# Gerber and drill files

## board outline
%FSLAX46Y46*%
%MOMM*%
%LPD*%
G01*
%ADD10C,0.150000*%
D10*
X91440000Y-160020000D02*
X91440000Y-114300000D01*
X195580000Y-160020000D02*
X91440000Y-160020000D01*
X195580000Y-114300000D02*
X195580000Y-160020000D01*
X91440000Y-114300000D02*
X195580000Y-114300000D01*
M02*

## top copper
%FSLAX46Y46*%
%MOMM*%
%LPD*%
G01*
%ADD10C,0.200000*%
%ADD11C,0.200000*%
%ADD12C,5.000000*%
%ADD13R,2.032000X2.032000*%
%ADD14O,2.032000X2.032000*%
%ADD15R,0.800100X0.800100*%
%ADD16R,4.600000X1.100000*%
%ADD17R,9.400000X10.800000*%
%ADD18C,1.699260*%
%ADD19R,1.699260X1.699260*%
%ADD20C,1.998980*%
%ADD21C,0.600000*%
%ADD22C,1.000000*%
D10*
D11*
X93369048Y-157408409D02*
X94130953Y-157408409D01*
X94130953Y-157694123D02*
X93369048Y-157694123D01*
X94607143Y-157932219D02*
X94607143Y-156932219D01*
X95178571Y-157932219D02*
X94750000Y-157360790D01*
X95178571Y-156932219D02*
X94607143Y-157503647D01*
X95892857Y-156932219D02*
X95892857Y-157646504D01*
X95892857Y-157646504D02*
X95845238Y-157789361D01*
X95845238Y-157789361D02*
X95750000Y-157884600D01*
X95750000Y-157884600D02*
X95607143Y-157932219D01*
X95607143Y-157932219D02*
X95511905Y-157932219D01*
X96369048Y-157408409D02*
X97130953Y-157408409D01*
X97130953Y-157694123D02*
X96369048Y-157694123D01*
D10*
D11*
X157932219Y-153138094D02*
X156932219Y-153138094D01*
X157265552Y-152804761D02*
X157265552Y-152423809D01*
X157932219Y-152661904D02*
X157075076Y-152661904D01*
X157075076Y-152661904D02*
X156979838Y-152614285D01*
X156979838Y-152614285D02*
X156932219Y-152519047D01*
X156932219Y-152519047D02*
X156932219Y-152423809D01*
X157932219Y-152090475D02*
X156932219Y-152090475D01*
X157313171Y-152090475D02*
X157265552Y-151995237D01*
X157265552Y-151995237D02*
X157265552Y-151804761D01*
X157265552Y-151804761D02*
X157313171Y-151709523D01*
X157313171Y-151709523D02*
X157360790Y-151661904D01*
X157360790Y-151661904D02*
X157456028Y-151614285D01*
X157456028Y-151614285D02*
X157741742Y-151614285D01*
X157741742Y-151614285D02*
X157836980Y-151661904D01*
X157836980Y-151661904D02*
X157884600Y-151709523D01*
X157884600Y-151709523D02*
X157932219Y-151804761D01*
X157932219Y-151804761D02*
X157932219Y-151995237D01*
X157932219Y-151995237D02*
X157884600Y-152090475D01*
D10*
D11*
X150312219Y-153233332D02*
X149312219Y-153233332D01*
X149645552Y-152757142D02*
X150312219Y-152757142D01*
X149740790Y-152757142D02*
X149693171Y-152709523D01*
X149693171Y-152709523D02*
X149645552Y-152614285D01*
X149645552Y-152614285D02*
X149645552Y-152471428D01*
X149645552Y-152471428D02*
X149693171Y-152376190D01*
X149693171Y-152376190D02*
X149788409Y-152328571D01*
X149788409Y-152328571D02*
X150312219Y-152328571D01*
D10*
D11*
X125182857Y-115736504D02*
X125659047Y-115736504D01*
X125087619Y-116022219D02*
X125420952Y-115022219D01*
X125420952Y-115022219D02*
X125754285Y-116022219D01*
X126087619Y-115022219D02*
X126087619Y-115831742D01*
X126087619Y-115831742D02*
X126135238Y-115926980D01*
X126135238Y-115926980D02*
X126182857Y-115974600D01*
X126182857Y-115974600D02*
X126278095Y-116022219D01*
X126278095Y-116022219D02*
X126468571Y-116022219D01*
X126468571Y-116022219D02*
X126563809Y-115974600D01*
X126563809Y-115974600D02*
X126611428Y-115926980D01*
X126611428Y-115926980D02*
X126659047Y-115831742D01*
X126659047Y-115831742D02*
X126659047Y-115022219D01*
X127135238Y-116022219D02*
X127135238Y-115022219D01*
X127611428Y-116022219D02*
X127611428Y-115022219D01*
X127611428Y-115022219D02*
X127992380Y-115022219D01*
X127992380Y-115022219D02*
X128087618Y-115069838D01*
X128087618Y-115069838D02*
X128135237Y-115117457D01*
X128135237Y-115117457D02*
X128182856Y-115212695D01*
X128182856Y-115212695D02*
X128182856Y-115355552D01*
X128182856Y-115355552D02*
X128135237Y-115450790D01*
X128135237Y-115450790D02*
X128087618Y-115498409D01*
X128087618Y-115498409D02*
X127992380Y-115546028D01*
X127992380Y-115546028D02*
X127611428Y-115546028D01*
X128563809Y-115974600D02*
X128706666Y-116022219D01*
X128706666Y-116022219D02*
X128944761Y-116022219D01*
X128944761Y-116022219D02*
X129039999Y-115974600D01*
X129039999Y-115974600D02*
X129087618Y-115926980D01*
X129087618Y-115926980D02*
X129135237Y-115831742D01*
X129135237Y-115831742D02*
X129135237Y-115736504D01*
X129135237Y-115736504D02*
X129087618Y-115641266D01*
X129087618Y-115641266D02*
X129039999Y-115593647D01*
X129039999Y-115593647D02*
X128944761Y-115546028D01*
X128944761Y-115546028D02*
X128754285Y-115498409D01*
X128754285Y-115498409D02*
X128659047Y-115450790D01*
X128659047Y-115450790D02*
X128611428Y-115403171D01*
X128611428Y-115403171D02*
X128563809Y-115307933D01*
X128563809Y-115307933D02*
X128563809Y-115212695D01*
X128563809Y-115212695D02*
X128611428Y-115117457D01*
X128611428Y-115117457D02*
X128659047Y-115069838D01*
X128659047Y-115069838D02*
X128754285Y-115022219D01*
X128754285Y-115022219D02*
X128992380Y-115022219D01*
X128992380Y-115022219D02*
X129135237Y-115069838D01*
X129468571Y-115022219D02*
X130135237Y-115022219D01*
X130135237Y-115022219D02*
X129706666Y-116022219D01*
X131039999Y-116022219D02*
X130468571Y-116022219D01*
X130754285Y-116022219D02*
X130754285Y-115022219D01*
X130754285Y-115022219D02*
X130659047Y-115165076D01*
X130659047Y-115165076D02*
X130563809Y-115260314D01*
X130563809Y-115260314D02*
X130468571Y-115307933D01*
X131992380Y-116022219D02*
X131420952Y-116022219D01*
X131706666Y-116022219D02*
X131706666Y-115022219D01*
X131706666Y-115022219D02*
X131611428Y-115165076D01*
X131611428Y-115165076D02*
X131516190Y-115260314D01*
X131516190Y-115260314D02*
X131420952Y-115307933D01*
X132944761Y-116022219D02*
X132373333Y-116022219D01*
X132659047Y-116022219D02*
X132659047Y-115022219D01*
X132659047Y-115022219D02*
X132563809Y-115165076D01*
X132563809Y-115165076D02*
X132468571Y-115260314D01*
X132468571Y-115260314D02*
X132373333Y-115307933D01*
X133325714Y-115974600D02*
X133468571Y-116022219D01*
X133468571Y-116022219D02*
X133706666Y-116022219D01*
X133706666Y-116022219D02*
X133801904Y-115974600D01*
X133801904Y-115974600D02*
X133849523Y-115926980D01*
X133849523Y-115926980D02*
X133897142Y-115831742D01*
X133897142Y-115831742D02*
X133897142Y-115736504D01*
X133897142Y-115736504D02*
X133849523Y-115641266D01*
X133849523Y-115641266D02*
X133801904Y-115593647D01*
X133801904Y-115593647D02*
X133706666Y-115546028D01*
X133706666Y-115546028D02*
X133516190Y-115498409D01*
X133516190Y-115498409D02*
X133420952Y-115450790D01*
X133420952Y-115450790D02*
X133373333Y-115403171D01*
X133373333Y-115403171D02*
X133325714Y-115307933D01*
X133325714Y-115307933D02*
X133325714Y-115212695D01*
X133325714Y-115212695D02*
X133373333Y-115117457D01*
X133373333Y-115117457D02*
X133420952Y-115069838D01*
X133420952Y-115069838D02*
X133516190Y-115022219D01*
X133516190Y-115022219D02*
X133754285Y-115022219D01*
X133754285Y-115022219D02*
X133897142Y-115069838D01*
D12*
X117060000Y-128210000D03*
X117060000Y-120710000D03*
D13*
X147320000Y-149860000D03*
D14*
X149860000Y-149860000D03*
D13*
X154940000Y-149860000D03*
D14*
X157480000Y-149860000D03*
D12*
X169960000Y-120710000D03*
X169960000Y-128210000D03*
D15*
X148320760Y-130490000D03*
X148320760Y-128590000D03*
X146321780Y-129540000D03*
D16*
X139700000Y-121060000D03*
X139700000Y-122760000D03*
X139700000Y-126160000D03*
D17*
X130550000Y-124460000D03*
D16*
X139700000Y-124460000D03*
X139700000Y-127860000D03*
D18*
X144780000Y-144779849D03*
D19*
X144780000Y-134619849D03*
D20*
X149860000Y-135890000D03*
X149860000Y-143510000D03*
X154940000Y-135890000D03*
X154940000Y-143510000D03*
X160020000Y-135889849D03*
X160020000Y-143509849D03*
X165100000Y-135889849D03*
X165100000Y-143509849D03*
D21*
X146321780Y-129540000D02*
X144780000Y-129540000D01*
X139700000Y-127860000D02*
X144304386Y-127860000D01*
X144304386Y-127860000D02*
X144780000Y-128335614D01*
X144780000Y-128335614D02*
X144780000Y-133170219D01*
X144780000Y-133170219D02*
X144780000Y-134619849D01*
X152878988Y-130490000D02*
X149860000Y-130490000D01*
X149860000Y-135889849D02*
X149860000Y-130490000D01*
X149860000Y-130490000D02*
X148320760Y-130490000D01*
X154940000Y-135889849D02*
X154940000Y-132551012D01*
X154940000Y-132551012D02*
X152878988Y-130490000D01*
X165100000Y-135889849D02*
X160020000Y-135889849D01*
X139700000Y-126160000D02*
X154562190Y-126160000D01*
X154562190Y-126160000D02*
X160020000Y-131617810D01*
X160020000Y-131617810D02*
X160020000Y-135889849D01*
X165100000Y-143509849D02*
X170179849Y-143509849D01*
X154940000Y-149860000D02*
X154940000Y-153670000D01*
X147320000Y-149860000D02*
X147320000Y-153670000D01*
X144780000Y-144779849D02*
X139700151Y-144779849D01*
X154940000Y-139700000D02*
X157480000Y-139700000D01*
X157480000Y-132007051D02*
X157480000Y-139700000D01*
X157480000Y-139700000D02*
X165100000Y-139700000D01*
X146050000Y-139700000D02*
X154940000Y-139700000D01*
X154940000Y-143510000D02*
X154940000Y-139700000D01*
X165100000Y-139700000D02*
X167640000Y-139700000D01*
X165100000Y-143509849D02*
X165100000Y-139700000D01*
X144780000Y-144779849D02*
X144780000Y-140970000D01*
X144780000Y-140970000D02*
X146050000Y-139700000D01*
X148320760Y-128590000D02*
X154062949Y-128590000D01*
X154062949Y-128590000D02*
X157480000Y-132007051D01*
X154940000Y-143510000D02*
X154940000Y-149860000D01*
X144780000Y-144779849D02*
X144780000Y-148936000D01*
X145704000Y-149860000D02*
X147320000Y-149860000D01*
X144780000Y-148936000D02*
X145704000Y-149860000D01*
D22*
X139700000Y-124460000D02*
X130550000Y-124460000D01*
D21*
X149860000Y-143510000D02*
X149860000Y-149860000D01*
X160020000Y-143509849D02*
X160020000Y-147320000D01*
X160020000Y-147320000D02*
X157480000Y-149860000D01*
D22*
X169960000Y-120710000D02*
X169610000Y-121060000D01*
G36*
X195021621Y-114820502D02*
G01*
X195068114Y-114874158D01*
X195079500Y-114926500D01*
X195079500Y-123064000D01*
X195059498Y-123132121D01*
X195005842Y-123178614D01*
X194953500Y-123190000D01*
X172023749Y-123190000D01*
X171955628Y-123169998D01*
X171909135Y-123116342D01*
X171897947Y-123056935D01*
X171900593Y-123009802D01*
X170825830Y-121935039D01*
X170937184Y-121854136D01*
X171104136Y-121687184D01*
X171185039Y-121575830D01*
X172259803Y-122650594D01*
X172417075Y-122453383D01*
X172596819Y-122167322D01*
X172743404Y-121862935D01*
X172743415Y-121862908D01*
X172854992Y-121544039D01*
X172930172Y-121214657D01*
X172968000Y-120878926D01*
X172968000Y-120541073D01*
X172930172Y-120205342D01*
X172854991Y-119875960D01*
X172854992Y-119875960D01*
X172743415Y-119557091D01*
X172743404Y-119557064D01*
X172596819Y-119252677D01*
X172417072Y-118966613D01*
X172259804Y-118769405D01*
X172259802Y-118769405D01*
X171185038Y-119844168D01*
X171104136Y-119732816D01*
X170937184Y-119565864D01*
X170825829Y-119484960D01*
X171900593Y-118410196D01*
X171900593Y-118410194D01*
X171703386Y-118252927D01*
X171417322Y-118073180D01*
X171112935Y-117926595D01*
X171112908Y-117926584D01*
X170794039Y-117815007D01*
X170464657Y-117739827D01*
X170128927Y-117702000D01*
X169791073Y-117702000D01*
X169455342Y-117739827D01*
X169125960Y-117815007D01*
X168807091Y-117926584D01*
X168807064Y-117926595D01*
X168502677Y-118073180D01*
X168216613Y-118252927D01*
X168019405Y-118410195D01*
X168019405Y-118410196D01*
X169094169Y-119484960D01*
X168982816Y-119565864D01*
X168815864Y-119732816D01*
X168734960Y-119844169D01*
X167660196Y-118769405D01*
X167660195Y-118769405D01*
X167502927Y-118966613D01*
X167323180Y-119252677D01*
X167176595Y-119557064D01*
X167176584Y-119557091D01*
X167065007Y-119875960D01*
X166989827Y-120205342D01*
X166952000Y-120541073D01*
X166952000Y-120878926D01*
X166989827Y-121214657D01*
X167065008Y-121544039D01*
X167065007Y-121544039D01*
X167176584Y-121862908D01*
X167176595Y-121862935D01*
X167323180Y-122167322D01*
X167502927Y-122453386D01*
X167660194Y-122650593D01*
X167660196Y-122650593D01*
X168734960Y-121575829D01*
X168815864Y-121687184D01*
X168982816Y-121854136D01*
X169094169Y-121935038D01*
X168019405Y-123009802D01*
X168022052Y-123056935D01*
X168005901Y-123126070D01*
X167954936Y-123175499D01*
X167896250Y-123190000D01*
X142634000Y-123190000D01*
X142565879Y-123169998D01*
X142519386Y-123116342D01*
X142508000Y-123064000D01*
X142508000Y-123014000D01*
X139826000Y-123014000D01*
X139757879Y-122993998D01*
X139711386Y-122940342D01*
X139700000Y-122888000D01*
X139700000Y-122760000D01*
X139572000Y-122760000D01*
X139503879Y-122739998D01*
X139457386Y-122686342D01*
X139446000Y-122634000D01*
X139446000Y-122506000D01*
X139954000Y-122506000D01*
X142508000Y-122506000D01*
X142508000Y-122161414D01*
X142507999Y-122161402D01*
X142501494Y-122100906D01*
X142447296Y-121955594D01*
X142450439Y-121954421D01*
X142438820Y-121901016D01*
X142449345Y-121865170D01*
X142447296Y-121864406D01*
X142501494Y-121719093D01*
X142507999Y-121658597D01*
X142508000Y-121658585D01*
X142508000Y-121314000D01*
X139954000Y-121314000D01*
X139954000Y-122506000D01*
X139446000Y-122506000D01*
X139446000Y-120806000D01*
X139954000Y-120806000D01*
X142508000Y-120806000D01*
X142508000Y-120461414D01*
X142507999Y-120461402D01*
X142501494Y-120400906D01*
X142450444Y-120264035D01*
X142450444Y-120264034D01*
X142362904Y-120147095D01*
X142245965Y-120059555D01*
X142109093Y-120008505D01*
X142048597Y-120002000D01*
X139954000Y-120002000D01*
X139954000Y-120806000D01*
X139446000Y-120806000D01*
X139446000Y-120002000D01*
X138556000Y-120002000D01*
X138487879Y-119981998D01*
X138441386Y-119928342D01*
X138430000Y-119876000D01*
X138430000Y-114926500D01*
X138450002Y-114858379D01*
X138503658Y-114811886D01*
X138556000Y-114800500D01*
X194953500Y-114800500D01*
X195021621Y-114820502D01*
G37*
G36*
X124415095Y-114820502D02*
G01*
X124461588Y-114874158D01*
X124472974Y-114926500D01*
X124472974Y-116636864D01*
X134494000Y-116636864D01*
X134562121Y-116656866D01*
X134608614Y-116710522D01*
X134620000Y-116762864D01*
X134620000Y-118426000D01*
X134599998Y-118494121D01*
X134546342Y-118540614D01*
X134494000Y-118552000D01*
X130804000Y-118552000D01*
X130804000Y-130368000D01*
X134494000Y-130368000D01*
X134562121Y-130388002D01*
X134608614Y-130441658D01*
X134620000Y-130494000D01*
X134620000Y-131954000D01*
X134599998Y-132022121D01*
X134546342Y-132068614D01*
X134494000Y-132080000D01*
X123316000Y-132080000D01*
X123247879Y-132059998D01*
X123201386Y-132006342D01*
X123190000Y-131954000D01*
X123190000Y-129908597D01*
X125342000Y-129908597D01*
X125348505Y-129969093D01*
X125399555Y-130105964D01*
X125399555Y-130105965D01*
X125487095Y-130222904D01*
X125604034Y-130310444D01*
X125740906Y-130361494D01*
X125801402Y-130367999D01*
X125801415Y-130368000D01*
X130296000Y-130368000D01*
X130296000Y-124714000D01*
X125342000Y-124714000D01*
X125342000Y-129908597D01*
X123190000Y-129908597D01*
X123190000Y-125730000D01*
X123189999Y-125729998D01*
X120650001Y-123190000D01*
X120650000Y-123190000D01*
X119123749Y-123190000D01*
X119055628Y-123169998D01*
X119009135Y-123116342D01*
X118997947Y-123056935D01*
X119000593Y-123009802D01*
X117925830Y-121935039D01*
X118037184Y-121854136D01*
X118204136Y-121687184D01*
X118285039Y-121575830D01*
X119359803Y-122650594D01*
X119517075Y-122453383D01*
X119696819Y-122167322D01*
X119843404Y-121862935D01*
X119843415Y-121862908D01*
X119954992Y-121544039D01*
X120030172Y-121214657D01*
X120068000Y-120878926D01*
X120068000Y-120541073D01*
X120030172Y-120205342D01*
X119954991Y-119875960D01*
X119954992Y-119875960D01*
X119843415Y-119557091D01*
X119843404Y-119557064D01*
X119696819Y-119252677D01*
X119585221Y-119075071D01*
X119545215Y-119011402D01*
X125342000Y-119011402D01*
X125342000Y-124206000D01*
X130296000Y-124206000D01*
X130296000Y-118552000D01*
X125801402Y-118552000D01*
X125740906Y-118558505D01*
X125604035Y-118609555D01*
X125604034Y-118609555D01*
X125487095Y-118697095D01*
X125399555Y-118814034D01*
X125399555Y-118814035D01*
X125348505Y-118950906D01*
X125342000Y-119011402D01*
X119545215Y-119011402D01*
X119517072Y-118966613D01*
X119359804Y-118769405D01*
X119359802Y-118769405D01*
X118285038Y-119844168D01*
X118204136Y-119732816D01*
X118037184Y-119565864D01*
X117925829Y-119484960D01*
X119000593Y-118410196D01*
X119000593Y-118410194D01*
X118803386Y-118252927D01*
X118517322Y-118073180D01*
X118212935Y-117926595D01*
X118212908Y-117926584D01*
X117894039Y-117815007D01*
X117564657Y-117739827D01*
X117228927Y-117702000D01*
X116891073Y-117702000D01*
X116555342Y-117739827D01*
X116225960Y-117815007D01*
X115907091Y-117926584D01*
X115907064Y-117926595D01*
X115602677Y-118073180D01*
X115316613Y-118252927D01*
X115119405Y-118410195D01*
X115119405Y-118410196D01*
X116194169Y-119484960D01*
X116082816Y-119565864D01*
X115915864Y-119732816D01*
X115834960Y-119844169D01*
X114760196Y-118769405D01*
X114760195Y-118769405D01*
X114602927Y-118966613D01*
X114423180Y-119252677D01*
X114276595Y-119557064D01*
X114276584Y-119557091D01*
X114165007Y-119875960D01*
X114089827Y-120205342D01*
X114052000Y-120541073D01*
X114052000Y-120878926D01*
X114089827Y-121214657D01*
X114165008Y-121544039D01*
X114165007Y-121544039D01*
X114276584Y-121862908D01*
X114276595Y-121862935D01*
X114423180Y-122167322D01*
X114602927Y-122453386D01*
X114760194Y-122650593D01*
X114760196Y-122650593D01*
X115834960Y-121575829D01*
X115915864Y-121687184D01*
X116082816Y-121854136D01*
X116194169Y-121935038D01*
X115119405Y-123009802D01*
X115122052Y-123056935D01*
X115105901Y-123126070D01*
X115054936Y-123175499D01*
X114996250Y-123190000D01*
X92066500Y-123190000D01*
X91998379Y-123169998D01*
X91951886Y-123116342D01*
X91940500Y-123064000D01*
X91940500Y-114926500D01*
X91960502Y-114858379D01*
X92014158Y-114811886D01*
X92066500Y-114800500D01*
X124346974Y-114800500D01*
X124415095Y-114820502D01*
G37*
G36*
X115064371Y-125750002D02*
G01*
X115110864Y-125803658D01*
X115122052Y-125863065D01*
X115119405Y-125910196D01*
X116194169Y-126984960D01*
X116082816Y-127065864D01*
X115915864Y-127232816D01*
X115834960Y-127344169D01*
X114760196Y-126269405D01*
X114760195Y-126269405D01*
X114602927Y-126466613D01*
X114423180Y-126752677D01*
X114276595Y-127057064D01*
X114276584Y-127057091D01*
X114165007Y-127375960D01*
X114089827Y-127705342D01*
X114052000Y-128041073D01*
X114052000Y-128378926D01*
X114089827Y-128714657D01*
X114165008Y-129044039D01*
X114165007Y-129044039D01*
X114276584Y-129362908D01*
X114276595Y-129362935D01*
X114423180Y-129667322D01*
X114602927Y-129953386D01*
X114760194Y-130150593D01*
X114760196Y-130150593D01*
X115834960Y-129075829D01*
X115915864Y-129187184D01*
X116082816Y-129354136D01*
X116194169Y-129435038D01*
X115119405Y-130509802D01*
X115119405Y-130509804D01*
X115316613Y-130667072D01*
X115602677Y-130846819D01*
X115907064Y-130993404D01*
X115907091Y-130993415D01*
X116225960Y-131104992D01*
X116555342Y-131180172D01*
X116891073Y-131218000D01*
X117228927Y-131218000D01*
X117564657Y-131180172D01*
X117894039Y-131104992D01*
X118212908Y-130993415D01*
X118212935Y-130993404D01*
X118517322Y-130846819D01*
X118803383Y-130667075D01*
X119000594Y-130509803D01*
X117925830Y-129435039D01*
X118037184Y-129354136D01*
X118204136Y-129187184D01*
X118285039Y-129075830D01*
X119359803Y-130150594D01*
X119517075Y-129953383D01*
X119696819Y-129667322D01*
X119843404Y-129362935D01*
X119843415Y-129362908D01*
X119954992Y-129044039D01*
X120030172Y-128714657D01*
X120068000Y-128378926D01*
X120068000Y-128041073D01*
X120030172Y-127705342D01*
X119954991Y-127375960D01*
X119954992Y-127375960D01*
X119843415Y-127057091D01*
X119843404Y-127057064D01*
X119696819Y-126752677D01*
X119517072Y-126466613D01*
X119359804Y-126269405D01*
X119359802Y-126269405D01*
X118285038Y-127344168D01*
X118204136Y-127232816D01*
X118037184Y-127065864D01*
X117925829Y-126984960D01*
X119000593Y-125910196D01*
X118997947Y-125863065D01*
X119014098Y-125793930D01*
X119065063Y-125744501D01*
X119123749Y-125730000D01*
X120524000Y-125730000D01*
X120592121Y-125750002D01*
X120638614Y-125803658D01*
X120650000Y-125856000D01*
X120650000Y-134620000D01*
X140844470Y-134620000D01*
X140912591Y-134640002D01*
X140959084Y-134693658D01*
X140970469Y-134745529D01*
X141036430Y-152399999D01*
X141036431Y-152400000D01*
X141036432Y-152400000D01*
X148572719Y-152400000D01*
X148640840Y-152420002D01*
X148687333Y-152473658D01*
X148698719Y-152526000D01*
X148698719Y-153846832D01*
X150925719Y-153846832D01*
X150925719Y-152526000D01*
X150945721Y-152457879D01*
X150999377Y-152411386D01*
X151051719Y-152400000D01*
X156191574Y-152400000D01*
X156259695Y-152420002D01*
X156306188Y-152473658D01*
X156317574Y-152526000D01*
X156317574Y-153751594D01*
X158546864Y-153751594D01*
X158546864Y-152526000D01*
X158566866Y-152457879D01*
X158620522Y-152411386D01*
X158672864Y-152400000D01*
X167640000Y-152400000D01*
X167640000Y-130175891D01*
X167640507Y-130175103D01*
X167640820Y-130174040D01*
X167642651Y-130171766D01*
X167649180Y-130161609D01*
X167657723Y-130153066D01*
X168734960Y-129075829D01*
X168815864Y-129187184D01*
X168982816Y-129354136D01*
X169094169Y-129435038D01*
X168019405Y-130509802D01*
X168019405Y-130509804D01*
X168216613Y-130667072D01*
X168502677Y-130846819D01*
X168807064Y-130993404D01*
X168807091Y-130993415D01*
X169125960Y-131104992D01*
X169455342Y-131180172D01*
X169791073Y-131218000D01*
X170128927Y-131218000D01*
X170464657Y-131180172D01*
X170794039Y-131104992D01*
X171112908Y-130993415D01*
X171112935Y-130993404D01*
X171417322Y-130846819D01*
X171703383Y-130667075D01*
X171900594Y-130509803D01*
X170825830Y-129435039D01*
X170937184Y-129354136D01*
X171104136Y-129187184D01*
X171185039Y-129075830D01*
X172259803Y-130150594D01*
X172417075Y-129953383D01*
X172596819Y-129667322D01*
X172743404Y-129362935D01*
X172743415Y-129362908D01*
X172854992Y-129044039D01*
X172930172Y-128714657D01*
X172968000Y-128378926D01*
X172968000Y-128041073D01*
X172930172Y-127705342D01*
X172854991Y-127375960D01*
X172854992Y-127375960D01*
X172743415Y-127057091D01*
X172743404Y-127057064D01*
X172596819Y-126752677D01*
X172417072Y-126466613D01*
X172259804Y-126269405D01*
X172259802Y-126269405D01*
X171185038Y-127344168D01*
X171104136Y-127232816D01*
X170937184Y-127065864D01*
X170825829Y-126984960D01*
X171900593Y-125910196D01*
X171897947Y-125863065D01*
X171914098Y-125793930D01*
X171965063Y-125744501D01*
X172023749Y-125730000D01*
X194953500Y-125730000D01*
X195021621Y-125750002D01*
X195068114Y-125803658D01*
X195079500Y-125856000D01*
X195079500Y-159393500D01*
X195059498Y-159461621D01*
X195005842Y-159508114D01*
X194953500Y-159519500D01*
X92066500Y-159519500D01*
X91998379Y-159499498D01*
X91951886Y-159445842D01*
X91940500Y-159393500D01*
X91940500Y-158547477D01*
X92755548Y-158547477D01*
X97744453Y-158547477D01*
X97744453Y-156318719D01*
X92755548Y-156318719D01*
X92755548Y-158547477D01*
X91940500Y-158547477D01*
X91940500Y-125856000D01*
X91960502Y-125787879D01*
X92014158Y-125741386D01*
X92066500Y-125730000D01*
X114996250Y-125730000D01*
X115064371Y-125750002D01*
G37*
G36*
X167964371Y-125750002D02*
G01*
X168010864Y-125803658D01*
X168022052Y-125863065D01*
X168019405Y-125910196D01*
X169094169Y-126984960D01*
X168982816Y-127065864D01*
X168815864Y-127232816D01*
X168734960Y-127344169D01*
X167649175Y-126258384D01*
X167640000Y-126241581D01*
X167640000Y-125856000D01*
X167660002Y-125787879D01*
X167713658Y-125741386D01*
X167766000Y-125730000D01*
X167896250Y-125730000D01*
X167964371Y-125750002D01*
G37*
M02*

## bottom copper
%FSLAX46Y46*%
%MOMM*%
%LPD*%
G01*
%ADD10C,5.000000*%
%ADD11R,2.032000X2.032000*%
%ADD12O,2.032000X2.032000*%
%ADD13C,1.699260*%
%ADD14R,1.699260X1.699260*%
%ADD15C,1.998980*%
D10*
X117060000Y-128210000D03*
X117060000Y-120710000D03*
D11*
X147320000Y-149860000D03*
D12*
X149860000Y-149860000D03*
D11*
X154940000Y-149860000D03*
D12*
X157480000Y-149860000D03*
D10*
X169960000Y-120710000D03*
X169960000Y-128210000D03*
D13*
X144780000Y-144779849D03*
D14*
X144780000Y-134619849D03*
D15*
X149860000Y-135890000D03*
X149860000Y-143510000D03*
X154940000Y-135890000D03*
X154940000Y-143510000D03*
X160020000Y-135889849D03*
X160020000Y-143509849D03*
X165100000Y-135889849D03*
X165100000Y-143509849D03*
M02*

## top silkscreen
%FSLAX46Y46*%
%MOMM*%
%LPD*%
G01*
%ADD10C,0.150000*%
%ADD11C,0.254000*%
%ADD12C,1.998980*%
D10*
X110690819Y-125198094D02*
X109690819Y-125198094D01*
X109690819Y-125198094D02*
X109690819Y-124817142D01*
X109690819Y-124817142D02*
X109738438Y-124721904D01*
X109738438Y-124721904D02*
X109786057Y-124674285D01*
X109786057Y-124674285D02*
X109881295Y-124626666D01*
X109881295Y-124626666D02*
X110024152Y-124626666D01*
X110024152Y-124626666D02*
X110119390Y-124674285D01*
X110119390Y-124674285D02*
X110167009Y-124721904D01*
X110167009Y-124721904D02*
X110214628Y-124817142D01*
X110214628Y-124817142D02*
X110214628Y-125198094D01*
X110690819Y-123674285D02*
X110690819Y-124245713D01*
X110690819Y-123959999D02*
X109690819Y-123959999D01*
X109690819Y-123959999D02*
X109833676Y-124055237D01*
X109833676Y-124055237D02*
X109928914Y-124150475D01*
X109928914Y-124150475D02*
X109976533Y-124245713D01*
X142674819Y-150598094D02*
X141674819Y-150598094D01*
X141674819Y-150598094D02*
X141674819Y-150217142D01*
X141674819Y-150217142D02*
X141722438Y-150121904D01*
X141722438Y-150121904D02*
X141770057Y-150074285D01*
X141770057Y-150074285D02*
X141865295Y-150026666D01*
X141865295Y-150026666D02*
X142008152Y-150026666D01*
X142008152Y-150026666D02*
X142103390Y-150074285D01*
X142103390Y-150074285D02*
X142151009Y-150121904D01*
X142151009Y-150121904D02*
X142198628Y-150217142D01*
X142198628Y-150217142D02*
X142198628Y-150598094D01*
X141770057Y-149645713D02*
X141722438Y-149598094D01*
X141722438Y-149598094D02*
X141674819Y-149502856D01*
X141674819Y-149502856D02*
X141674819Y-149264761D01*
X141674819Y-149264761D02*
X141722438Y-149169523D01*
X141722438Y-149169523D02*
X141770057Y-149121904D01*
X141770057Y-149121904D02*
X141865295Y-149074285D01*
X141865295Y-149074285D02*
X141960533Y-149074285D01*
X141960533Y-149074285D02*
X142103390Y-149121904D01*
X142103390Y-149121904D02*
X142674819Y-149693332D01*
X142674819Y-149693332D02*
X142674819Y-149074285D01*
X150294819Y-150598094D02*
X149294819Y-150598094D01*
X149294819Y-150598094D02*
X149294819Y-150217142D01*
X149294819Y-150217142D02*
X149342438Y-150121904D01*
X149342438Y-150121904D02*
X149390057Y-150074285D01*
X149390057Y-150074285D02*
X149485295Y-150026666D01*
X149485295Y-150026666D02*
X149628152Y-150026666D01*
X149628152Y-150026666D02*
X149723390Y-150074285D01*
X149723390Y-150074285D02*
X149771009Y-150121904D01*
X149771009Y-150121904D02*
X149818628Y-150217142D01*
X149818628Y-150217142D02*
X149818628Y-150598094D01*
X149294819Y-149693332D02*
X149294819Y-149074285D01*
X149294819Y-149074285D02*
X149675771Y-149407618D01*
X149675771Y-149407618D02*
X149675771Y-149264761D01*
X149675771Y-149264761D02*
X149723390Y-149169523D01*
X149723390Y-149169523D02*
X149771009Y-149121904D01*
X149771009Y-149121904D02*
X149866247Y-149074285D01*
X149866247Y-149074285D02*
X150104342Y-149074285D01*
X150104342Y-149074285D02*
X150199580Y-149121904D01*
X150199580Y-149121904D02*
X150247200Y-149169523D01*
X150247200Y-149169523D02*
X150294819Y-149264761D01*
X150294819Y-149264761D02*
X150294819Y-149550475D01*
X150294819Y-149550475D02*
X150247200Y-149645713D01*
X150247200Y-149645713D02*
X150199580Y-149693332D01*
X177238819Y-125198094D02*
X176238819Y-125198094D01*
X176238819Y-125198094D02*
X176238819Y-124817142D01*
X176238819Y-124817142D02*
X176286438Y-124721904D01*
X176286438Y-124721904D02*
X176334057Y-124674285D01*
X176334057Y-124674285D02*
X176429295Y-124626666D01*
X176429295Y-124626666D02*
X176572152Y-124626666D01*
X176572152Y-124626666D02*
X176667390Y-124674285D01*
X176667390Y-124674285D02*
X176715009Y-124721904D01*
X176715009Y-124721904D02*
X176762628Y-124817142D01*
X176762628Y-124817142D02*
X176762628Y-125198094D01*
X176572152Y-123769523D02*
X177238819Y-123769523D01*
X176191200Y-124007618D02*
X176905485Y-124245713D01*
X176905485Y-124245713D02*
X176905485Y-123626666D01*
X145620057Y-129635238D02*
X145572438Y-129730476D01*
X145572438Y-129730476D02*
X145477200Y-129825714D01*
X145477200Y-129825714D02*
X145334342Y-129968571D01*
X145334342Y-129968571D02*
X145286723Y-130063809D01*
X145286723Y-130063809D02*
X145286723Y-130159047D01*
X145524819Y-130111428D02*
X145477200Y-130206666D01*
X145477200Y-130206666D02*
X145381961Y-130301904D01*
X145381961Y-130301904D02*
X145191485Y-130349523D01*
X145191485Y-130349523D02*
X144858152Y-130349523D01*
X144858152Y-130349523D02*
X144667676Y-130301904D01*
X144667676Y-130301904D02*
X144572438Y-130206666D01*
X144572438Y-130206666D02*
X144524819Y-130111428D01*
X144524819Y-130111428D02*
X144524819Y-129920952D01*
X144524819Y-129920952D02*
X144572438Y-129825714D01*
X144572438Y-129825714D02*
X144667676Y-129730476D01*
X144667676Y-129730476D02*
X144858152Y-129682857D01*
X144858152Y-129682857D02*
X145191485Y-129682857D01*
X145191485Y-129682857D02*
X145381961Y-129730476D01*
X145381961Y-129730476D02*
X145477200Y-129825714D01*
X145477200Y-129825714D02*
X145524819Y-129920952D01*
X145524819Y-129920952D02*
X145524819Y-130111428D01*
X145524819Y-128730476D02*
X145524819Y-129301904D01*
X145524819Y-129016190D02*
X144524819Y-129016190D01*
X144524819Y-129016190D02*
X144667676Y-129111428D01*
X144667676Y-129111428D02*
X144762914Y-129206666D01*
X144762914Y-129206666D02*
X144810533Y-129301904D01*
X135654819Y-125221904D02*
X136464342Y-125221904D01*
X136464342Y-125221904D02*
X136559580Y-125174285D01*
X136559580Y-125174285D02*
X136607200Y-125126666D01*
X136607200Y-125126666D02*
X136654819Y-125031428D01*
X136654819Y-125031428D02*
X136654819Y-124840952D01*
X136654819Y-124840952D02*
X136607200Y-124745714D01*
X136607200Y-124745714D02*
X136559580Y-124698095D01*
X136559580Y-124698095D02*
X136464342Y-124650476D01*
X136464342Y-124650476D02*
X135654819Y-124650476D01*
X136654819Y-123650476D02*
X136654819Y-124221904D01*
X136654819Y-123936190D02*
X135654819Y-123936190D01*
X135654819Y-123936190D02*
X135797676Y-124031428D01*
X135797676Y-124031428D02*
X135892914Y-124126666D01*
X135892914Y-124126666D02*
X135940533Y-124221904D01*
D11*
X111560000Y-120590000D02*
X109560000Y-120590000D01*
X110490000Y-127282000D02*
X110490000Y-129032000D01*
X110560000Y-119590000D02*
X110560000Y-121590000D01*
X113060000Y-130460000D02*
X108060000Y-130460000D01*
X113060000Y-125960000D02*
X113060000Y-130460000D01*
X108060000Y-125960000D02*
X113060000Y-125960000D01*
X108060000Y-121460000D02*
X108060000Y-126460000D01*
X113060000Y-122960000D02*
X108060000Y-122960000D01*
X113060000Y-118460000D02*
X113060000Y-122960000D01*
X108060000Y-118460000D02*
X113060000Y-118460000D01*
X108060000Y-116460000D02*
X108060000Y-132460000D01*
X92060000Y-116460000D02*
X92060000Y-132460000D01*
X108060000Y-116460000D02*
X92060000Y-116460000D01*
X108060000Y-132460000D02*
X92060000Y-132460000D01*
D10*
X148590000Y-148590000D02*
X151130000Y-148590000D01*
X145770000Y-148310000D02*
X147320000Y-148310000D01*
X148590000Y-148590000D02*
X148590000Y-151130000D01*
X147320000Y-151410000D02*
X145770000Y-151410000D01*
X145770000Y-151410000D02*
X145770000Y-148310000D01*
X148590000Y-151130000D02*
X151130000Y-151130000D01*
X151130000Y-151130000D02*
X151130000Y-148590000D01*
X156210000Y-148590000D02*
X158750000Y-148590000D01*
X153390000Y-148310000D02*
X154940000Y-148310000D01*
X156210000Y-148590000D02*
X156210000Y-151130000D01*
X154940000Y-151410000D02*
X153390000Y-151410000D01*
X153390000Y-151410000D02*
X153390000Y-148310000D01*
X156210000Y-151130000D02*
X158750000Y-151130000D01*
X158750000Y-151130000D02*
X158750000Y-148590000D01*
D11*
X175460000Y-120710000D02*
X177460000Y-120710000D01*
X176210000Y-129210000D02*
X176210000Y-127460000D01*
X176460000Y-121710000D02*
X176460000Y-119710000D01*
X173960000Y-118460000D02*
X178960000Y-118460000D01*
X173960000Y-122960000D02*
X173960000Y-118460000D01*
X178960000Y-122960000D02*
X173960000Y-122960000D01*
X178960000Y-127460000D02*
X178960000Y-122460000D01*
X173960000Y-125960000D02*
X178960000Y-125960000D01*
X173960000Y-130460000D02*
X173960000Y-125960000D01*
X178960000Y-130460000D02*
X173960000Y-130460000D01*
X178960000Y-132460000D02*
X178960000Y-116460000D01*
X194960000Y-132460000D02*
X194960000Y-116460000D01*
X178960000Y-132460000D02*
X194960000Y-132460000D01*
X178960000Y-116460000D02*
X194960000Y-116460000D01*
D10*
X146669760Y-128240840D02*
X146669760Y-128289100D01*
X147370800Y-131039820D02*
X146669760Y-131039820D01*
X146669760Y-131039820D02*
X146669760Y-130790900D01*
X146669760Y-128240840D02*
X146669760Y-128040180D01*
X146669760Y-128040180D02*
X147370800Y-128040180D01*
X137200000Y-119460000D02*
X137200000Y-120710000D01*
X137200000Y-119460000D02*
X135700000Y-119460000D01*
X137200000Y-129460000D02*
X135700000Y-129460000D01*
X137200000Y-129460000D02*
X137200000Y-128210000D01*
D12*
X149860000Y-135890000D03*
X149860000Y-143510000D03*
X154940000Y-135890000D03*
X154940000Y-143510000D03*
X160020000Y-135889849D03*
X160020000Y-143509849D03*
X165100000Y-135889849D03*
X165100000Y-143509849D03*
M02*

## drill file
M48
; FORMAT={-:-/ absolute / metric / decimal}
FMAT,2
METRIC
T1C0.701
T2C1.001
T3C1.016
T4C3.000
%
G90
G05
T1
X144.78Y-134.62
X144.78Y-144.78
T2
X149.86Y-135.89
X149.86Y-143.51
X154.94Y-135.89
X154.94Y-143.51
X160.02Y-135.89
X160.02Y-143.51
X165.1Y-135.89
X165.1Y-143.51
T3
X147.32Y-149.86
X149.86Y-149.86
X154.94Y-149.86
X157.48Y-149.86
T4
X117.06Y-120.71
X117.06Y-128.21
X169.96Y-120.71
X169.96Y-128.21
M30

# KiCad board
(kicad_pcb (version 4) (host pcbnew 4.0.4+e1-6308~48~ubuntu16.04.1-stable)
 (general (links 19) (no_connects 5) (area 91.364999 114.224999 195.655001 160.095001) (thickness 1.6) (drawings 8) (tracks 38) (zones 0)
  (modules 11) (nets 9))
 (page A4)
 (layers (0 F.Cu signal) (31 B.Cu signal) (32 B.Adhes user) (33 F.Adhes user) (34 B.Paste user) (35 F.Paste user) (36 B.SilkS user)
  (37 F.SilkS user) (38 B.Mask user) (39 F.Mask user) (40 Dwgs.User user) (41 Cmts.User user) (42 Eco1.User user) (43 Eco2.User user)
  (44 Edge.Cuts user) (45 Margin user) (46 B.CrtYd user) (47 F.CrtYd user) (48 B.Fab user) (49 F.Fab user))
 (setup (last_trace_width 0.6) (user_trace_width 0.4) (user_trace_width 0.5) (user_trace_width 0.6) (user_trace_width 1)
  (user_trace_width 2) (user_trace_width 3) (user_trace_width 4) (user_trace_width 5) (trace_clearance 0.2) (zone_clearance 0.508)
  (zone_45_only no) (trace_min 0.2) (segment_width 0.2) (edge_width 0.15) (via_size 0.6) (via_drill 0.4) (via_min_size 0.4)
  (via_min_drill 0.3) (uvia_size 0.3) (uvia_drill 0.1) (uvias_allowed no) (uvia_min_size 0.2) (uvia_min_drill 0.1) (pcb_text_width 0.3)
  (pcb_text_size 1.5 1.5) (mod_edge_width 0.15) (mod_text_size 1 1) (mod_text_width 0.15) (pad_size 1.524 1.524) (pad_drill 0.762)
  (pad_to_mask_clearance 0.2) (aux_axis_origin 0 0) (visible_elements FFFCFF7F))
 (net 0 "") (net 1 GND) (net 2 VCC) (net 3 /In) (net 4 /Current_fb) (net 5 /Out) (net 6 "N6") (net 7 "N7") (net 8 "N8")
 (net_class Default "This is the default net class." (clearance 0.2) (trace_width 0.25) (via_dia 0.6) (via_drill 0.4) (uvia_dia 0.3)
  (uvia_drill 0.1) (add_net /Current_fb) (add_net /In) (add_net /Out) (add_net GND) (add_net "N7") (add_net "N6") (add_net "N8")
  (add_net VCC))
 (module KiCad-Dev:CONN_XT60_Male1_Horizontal (layer F.Cu) (at 99.06 124.46 270)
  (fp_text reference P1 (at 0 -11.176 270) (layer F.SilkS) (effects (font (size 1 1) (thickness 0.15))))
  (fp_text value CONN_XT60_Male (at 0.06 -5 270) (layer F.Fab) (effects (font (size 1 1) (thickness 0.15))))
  (fp_line (start -3.87 -12.5) (end -3.87 -10.5) (layer F.SilkS) (width 0.254))
  (fp_line (start 2.822 -11.43) (end 4.572 -11.43) (layer F.SilkS) (width 0.254))
  (fp_line (start -4.87 -11.5) (end -2.87 -11.5) (layer F.SilkS) (width 0.254))
  (fp_line (start 6 -14) (end 6 -9) (layer F.SilkS) (width 0.254))
  (fp_line (start 1.5 -14) (end 6 -14) (layer F.SilkS) (width 0.254))
  (fp_line (start 1.5 -9) (end 1.5 -14) (layer F.SilkS) (width 0.254))
  (fp_line (start -3 -9) (end 2 -9) (layer F.SilkS) (width 0.254))
  (fp_line (start -1.5 -14) (end -1.5 -9) (layer F.SilkS) (width 0.254))
  (fp_line (start -6 -14) (end -1.5 -14) (layer F.SilkS) (width 0.254))
  (fp_line (start -6 -9) (end -6 -14) (layer F.SilkS) (width 0.254))
  (fp_line (start -8 -9) (end 8 -9) (layer F.SilkS) (width 0.254))
  (fp_line (start -8 7) (end 8 7) (layer F.SilkS) (width 0.254))
  (fp_line (start -8 -9) (end -8 7) (layer F.SilkS) (width 0.254))
  (fp_line (start 8 -9) (end 8 7) (layer F.SilkS) (width 0.254))
  (pad 1 thru_hole circle (at 3.75 -18 270) (size 5 5) (drill 3) (layers *.Cu *.Mask) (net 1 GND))
  (pad 2 thru_hole circle (at -3.75 -18 270) (size 5 5) (drill 3) (layers *.Cu *.Mask) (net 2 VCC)))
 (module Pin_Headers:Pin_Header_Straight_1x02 (layer F.Cu) (at 147.32 149.86 90)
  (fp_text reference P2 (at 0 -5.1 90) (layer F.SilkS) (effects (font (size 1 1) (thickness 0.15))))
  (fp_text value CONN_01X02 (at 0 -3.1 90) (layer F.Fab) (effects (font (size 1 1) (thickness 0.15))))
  (fp_line (start 1.27 1.27) (end 1.27 3.81) (layer F.SilkS) (width 0.15))
  (fp_line (start 1.55 -1.55) (end 1.55 0) (layer F.SilkS) (width 0.15))
  (fp_line (start 1.27 1.27) (end -1.27 1.27) (layer F.SilkS) (width 0.15))
  (fp_line (start -1.55 0) (end -1.55 -1.55) (layer F.SilkS) (width 0.15))
  (fp_line (start -1.55 -1.55) (end 1.55 -1.55) (layer F.SilkS) (width 0.15))
  (fp_line (start -1.27 1.27) (end -1.27 3.81) (layer F.SilkS) (width 0.15))
  (fp_line (start -1.27 3.81) (end 1.27 3.81) (layer F.SilkS) (width 0.15))
  (pad 1 thru_hole rect (at 0 0 90) (size 2.032 2.032) (drill 1.016) (layers *.Cu *.Mask) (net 1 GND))
  (pad 2 thru_hole oval (at 0 2.54 90) (size 2.032 2.032) (drill 1.016) (layers *.Cu *.Mask) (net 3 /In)))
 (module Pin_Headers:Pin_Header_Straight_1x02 (layer F.Cu) (at 154.94 149.86 90)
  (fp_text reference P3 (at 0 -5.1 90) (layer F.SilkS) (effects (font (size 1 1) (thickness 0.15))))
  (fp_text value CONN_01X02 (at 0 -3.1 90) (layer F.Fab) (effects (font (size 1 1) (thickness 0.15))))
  (fp_line (start 1.27 1.27) (end 1.27 3.81) (layer F.SilkS) (width 0.15))
  (fp_line (start 1.55 -1.55) (end 1.55 0) (layer F.SilkS) (width 0.15))
  (fp_line (start 1.27 1.27) (end -1.27 1.27) (layer F.SilkS) (width 0.15))
  (fp_line (start -1.55 0) (end -1.55 -1.55) (layer F.SilkS) (width 0.15))
  (fp_line (start -1.55 -1.55) (end 1.55 -1.55) (layer F.SilkS) (width 0.15))
  (fp_line (start -1.27 1.27) (end -1.27 3.81) (layer F.SilkS) (width 0.15))
  (fp_line (start -1.27 3.81) (end 1.27 3.81) (layer F.SilkS) (width 0.15))
  (pad 1 thru_hole rect (at 0 0 90) (size 2.032 2.032) (drill 1.016) (layers *.Cu *.Mask) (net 1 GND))
  (pad 2 thru_hole oval (at 0 2.54 90) (size 2.032 2.032) (drill 1.016) (layers *.Cu *.Mask) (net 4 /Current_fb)))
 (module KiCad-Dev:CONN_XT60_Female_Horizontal (layer F.Cu) (at 187.96 124.46 90)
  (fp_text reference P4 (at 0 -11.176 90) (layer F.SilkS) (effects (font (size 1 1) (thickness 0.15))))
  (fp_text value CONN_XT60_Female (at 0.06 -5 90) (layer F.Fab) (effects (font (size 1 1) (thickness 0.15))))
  (fp_line (start 3.75 -12.5) (end 3.75 -10.5) (layer F.SilkS) (width 0.254))
  (fp_line (start -4.75 -11.75) (end -3 -11.75) (layer F.SilkS) (width 0.254))
  (fp_line (start 2.75 -11.5) (end 4.75 -11.5) (layer F.SilkS) (width 0.254))
  (fp_line (start 6 -14) (end 6 -9) (layer F.SilkS) (width 0.254))
  (fp_line (start 1.5 -14) (end 6 -14) (layer F.SilkS) (width 0.254))
  (fp_line (start 1.5 -9) (end 1.5 -14) (layer F.SilkS) (width 0.254))
  (fp_line (start -3 -9) (end 2 -9) (layer F.SilkS) (width 0.254))
  (fp_line (start -1.5 -14) (end -1.5 -9) (layer F.SilkS) (width 0.254))
  (fp_line (start -6 -14) (end -1.5 -14) (layer F.SilkS) (width 0.254))
  (fp_line (start -6 -9) (end -6 -14) (layer F.SilkS) (width 0.254))
  (fp_line (start -8 -9) (end 8 -9) (layer F.SilkS) (width 0.254))
  (fp_line (start -8 7) (end 8 7) (layer F.SilkS) (width 0.254))
  (fp_line (start -8 -9) (end -8 7) (layer F.SilkS) (width 0.254))
  (fp_line (start 8 -9) (end 8 7) (layer F.SilkS) (width 0.254))
  (pad 2 thru_hole circle (at 3.75 -18 90) (size 5 5) (drill 3) (layers *.Cu *.Mask) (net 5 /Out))
  (pad 1 thru_hole circle (at -3.75 -18 90) (size 5 5) (drill 3) (layers *.Cu *.Mask) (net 1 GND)))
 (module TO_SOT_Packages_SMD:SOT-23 (layer F.Cu) (at 147.32 129.54 90)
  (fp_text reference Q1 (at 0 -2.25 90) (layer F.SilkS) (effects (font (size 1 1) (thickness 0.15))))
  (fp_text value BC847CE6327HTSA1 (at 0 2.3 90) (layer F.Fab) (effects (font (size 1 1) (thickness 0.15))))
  (fp_line (start 1.29916 -0.65024) (end 1.2509 -0.65024) (layer F.SilkS) (width 0.15))
  (fp_line (start -1.49982 0.0508) (end -1.49982 -0.65024) (layer F.SilkS) (width 0.15))
  (fp_line (start -1.49982 -0.65024) (end -1.2509 -0.65024) (layer F.SilkS) (width 0.15))
  (fp_line (start 1.29916 -0.65024) (end 1.49982 -0.65024) (layer F.SilkS) (width 0.15))
  (fp_line (start 1.49982 -0.65024) (end 1.49982 0.0508) (layer F.SilkS) (width 0.15))
  (pad 1 smd rect (at -0.95 1.00076 90) (size 0.8001 0.8001) (layers F.Cu F.Paste F.Mask) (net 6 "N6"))
  (pad 2 smd rect (at 0.95 1.00076 90) (size 0.8001 0.8001) (layers F.Cu F.Paste F.Mask) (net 1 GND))
  (pad 3 smd rect (at 0 -0.99822 90) (size 0.8001 0.8001) (layers F.Cu F.Paste F.Mask) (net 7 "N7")))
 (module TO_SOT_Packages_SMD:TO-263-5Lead (layer F.Cu) (at 139.7 124.46 180)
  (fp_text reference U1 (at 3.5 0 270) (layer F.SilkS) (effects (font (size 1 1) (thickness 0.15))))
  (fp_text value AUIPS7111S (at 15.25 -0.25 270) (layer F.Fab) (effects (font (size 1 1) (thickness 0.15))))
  (fp_line (start 2.5 5) (end 2.5 3.75) (layer F.SilkS) (width 0.15))
  (fp_line (start 2.5 5) (end 4 5) (layer F.SilkS) (width 0.15))
  (fp_line (start 2.5 -5) (end 4 -5) (layer F.SilkS) (width 0.15))
  (fp_line (start 2.5 -5) (end 2.5 -3.75) (layer F.SilkS) (width 0.15))
  (pad 5 smd rect (at 0 3.4 180) (size 4.6 1.1) (layers F.Cu F.Paste F.Mask) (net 5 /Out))
  (pad 4 smd rect (at 0 1.7 180) (size 4.6 1.1) (layers F.Cu F.Paste F.Mask) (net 5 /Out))
  (pad 2 smd rect (at 0 -1.7 180) (size 4.6 1.1) (layers F.Cu F.Paste F.Mask) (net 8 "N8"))
  (pad 3 smd rect (at 9.15 0 180) (size 9.4 10.8) (layers F.Cu F.Paste F.Mask) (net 2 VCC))
  (pad 3 smd rect (at 0 0 180) (size 4.6 1.1) (layers F.Cu F.Paste F.Mask) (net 2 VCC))
  (pad 1 smd rect (at 0 -3.4 180) (size 4.6 1.1) (layers F.Cu F.Paste F.Mask) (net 7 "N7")))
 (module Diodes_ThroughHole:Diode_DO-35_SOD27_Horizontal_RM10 (layer B.Cu) (at 144.78254 134.619329 270)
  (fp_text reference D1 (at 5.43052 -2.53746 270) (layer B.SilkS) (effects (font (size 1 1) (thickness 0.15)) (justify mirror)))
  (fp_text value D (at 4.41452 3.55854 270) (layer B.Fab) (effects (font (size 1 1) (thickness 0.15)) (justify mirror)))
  (pad 2 thru_hole circle (at 10.16052 0.00254 90) (size 1.69926 1.69926) (drill 0.70104) (layers *.Cu *.Mask) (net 1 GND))
  (pad 1 thru_hole rect (at 0.00052 0.00254 90) (size 1.69926 1.69926) (drill 0.70104) (layers *.Cu *.Mask) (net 7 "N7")))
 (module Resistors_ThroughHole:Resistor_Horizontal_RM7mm (layer B.Cu) (at 149.86 135.89 270)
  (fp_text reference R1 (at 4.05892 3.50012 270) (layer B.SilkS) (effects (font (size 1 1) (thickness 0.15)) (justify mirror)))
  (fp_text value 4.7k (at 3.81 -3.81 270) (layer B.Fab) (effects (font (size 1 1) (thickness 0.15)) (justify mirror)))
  (pad 1 thru_hole circle (at 0 0 270) (size 1.99898 1.99898) (drill 1.00076) (layers *.Cu *.SilkS *.Mask) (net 6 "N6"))
  (pad 2 thru_hole circle (at 7.62 0 270) (size 1.99898 1.99898) (drill 1.00076) (layers *.Cu *.SilkS *.Mask) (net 3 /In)))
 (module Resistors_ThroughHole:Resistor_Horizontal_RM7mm (layer B.Cu) (at 154.94 135.89 270)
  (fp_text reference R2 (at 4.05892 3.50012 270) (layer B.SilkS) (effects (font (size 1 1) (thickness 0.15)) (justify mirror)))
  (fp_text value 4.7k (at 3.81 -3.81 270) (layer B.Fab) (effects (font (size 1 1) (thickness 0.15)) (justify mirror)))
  (pad 1 thru_hole circle (at 0 0 270) (size 1.99898 1.99898) (drill 1.00076) (layers *.Cu *.SilkS *.Mask) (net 6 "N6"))
  (pad 2 thru_hole circle (at 7.62 0 270) (size 1.99898 1.99898) (drill 1.00076) (layers *.Cu *.SilkS *.Mask) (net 1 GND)))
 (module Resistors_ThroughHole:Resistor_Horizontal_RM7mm (layer B.Cu) (at 160.02 135.889849 270)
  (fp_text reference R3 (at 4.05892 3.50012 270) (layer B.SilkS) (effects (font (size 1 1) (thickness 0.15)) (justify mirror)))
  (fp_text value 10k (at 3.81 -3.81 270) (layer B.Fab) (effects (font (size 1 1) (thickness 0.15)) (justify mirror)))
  (pad 1 thru_hole circle (at 0 0 270) (size 1.99898 1.99898) (drill 1.00076) (layers *.Cu *.SilkS *.Mask) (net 8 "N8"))
  (pad 2 thru_hole circle (at 7.62 0 270) (size 1.99898 1.99898) (drill 1.00076) (layers *.Cu *.SilkS *.Mask) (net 4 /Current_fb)))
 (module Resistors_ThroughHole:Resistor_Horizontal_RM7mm (layer B.Cu) (at 165.1 135.889849 270)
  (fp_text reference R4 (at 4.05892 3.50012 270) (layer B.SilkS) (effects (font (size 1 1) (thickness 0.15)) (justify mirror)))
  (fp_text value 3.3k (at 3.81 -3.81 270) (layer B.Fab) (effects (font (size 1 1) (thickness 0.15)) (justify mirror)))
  (pad 1 thru_hole circle (at 0 0 270) (size 1.99898 1.99898) (drill 1.00076) (layers *.Cu *.SilkS *.Mask) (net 8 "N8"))
  (pad 2 thru_hole circle (at 7.62 0 270) (size 1.99898 1.99898) (drill 1.00076) (layers *.Cu *.SilkS *.Mask) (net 1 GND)))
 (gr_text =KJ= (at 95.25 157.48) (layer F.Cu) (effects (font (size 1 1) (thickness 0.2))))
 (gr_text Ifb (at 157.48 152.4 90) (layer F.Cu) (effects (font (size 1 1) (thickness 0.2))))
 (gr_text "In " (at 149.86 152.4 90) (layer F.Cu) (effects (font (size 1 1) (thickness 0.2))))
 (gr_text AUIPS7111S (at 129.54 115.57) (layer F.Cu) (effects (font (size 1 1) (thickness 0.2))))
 (gr_line (start 91.44 160.02) (end 91.44 114.3) (layer Edge.Cuts) (width 0.15))
 (gr_line (start 195.58 160.02) (end 91.44 160.02) (layer Edge.Cuts) (width 0.15))
 (gr_line (start 195.58 114.3) (end 195.58 160.02) (layer Edge.Cuts) (width 0.15))
 (gr_line (start 91.44 114.3) (end 195.58 114.3) (layer Edge.Cuts) (width 0.15))
 (segment (start 146.32178 129.54) (end 144.78 129.54) (width 0.6) (layer F.Cu) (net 7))
 (segment (start 139.7 127.86) (end 144.304386 127.86) (width 0.6) (layer F.Cu) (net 7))
 (segment (start 144.304386 127.86) (end 144.78 128.335614) (width 0.6) (layer F.Cu) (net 7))
 (segment (start 144.78 128.335614) (end 144.78 133.170219) (width 0.6) (layer F.Cu) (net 7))
 (segment (start 144.78 133.170219) (end 144.78 134.619849) (width 0.6) (layer F.Cu) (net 7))
 (segment (start 152.878988 130.49) (end 149.86 130.49) (width 0.6) (layer F.Cu) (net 6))
 (segment (start 149.86 135.889849) (end 149.86 130.49) (width 0.6) (layer F.Cu) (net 6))
 (segment (start 149.86 130.49) (end 148.32076 130.49) (width 0.6) (layer F.Cu) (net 6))
 (segment (start 154.94 135.889849) (end 154.94 132.551012) (width 0.6) (layer F.Cu) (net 6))
 (segment (start 154.94 132.551012) (end 152.878988 130.49) (width 0.6) (layer F.Cu) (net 6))
 (segment (start 165.1 135.889849) (end 160.02 135.889849) (width 0.6) (layer F.Cu) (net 8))
 (segment (start 139.7 126.16) (end 154.56219 126.16) (width 0.6) (layer F.Cu) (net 8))
 (segment (start 154.56219 126.16) (end 160.02 131.61781) (width 0.6) (layer F.Cu) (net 8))
 (segment (start 160.02 131.61781) (end 160.02 135.889849) (width 0.6) (layer F.Cu) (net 8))
 (segment (start 165.1 143.509849) (end 170.179849 143.509849) (width 0.6) (layer F.Cu) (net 1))
 (segment (start 154.94 149.86) (end 154.94 153.67) (width 0.6) (layer F.Cu) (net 1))
 (segment (start 147.32 149.86) (end 147.32 153.67) (width 0.6) (layer F.Cu) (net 1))
 (segment (start 144.78 144.779849) (end 139.700151 144.779849) (width 0.6) (layer F.Cu) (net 1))
 (segment (start 154.94 139.7) (end 157.48 139.7) (width 0.6) (layer F.Cu) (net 1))
 (segment (start 157.48 132.007051) (end 157.48 139.7) (width 0.6) (layer F.Cu) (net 1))
 (segment (start 157.48 139.7) (end 165.1 139.7) (width 0.6) (layer F.Cu) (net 1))
 (segment (start 146.05 139.7) (end 154.94 139.7) (width 0.6) (layer F.Cu) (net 1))
 (segment (start 154.94 143.51) (end 154.94 139.7) (width 0.6) (layer F.Cu) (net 1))
 (segment (start 165.1 139.7) (end 167.64 139.7) (width 0.6) (layer F.Cu) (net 1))
 (segment (start 165.1 143.509849) (end 165.1 139.7) (width 0.6) (layer F.Cu) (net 1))
 (segment (start 144.78 144.779849) (end 144.78 140.97) (width 0.6) (layer F.Cu) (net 1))
 (segment (start 144.78 140.97) (end 146.05 139.7) (width 0.6) (layer F.Cu) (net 1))
 (segment (start 148.32076 128.59) (end 154.062949 128.59) (width 0.6) (layer F.Cu) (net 1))
 (segment (start 154.062949 128.59) (end 157.48 132.007051) (width 0.6) (layer F.Cu) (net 1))
 (segment (start 154.94 143.51) (end 154.94 149.86) (width 0.6) (layer F.Cu) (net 1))
 (segment (start 144.78 144.779849) (end 144.78 148.936) (width 0.6) (layer F.Cu) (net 1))
 (segment (start 145.704 149.86) (end 147.32 149.86) (width 0.6) (layer F.Cu) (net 1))
 (segment (start 144.78 148.936) (end 145.704 149.86) (width 0.6) (layer F.Cu) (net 1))
 (segment (start 139.7 124.46) (end 130.55 124.46) (width 1) (layer F.Cu) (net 2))
 (segment (start 149.86 143.51) (end 149.86 149.86) (width 0.6) (layer F.Cu) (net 3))
 (segment (start 160.02 143.509849) (end 160.02 147.32) (width 0.6) (layer F.Cu) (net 4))
 (segment (start 160.02 147.32) (end 157.48 149.86) (width 0.6) (layer F.Cu) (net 4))
 (segment (start 169.96 120.71) (end 169.61 121.06) (width 1) (layer F.Cu) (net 5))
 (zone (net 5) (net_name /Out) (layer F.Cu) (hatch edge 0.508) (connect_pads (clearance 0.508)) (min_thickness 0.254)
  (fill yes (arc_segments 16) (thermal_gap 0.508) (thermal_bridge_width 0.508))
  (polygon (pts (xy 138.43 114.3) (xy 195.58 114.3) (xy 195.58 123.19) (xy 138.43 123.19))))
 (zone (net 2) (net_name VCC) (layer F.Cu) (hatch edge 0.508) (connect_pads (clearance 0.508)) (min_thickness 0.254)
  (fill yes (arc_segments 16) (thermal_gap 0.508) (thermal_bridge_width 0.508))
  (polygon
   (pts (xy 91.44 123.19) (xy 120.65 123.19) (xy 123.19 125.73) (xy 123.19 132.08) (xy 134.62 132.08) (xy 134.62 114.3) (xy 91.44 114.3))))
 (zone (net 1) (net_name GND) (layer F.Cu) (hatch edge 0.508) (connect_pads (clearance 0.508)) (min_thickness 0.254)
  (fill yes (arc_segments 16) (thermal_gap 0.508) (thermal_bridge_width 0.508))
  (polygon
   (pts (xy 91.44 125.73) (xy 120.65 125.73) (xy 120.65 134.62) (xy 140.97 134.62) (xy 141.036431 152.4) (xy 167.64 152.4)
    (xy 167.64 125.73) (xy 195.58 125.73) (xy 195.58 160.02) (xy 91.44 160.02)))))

